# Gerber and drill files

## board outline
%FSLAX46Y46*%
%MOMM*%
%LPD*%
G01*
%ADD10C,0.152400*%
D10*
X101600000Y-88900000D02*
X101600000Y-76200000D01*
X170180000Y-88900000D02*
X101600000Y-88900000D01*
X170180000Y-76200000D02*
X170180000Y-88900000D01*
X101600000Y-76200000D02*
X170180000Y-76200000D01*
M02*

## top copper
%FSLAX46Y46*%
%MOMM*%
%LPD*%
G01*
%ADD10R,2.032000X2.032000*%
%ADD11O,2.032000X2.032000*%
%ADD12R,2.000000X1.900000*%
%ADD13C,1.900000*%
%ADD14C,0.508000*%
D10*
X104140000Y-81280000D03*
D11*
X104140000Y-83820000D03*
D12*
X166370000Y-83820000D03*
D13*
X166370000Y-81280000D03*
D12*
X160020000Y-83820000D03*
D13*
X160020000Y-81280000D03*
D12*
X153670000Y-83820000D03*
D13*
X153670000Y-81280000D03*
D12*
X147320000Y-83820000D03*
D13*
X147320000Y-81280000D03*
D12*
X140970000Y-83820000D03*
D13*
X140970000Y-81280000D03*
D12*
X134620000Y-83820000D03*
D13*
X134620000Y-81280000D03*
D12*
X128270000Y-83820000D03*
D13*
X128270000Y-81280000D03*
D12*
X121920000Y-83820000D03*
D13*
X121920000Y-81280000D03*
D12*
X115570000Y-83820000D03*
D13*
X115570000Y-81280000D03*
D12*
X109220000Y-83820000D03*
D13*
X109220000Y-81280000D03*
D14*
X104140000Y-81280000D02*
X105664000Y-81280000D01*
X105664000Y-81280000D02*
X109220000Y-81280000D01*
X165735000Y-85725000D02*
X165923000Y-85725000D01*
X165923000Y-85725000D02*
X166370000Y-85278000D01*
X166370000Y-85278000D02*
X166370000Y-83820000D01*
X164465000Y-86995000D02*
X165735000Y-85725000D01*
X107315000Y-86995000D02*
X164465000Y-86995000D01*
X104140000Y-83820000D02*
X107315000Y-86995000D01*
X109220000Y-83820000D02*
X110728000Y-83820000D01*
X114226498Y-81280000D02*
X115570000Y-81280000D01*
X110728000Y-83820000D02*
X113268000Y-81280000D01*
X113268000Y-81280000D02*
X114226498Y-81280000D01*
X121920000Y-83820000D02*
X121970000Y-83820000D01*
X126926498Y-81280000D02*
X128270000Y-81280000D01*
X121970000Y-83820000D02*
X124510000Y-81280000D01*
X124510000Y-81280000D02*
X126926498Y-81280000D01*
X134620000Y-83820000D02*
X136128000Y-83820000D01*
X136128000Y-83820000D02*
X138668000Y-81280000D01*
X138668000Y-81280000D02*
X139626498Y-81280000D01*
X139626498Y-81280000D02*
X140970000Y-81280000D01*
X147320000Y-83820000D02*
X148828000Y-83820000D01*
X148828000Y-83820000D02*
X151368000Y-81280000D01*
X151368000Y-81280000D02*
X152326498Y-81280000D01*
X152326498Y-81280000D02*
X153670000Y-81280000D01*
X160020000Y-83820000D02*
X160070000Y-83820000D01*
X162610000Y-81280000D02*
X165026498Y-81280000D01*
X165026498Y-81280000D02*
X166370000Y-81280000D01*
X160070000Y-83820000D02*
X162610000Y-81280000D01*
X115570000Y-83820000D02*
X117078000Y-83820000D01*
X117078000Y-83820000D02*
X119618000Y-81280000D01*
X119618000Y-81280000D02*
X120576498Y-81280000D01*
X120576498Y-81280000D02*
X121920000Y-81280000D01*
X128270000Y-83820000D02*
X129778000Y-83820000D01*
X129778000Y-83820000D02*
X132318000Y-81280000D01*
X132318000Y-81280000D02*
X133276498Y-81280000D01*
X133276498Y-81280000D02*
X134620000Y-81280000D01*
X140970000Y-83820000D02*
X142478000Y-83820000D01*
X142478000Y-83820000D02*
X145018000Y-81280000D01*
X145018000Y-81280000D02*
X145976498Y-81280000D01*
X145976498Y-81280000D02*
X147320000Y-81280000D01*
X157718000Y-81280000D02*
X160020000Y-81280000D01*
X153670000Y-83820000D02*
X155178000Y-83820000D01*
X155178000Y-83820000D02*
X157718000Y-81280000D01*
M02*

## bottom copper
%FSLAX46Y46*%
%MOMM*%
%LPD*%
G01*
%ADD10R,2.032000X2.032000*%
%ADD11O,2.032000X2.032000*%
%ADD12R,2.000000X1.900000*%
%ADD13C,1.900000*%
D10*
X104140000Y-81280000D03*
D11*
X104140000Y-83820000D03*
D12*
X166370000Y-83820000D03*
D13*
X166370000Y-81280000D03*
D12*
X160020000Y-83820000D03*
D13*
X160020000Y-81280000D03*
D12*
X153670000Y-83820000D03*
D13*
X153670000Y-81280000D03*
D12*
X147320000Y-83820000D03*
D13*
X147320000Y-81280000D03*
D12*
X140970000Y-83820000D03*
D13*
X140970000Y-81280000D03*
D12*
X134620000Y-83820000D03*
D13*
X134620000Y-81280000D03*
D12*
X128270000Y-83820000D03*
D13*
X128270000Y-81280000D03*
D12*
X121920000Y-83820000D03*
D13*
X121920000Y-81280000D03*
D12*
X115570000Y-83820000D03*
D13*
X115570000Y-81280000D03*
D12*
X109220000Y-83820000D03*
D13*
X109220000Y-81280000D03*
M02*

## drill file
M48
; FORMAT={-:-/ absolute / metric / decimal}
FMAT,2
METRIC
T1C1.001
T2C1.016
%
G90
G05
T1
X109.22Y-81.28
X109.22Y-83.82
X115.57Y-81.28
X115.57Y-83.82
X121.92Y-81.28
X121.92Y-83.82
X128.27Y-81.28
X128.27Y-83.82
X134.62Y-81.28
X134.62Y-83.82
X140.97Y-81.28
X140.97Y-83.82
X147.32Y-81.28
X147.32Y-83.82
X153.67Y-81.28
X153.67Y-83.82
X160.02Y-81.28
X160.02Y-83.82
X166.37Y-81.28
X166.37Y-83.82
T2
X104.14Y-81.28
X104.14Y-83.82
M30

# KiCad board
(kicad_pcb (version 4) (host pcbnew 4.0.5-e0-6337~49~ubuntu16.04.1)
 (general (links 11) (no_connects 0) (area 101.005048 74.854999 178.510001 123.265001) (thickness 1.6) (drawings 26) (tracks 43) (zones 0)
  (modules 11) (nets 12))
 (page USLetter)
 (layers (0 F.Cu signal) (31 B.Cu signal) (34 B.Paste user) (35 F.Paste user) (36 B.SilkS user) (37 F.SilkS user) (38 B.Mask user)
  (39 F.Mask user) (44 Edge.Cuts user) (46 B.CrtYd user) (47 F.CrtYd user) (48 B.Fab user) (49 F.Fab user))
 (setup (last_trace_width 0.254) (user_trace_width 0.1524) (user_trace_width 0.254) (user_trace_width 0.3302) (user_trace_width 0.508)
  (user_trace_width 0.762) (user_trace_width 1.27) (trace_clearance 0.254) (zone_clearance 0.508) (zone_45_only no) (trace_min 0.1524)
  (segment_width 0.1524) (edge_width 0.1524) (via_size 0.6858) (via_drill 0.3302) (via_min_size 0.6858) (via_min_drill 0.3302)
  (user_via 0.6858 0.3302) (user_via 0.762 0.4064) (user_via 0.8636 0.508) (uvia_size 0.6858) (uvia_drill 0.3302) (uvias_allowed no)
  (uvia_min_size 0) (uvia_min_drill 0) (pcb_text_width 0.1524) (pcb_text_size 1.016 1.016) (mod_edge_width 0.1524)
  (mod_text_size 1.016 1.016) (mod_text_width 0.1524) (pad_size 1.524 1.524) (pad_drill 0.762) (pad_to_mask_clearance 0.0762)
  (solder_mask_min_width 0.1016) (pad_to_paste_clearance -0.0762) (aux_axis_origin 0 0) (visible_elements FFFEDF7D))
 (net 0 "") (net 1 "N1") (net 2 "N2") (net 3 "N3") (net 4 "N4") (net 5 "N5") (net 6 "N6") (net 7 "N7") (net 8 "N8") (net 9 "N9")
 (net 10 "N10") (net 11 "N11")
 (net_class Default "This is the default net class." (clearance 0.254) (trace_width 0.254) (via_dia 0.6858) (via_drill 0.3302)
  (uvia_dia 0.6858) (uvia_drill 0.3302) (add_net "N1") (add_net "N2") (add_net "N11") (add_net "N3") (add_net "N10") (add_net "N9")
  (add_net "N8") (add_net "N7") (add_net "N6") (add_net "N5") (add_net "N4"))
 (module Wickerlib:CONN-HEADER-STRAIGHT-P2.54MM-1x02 (layer F.Cu) (at 104.14 81.28)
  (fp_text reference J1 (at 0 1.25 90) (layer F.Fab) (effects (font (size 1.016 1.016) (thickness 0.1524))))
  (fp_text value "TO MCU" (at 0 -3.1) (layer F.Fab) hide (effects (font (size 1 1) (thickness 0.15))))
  (pad 1 thru_hole rect (at 0 0) (size 2.032 2.032) (drill 1.016) (layers *.Cu *.Mask F.SilkS) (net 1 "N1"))
  (pad 2 thru_hole oval (at 0 2.54) (size 2.032 2.032) (drill 1.016) (layers *.Cu *.Mask F.SilkS) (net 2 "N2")))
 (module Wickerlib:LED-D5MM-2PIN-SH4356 (layer F.Cu) (at 166.37 83.82 90)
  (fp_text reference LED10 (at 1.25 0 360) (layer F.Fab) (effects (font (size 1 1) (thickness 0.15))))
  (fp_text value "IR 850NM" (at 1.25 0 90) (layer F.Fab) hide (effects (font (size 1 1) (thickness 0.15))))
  (pad 1 thru_hole rect (at 0 0 180) (size 2 1.9) (drill 1.00076) (layers *.Cu *.Mask F.SilkS) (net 2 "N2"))
  (pad 2 thru_hole circle (at 2.54 0 90) (size 1.9 1.9) (drill 1.00076) (layers *.Cu *.Mask F.SilkS) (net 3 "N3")))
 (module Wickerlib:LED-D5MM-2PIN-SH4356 (layer F.Cu) (at 160.02 83.82 90)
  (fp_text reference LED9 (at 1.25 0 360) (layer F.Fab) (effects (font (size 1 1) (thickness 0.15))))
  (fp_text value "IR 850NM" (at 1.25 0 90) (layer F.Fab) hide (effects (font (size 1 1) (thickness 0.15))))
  (pad 1 thru_hole rect (at 0 0 180) (size 2 1.9) (drill 1.00076) (layers *.Cu *.Mask F.SilkS) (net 3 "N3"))
  (pad 2 thru_hole circle (at 2.54 0 90) (size 1.9 1.9) (drill 1.00076) (layers *.Cu *.Mask F.SilkS) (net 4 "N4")))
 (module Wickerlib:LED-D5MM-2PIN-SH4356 (layer F.Cu) (at 153.67 83.82 90)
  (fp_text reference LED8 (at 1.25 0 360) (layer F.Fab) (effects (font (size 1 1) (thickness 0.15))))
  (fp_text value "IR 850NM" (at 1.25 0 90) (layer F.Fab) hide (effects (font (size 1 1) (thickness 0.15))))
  (pad 1 thru_hole rect (at 0 0 180) (size 2 1.9) (drill 1.00076) (layers *.Cu *.Mask F.SilkS) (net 4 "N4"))
  (pad 2 thru_hole circle (at 2.54 0 90) (size 1.9 1.9) (drill 1.00076) (layers *.Cu *.Mask F.SilkS) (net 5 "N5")))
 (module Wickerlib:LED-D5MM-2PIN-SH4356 (layer F.Cu) (at 147.32 83.82 90)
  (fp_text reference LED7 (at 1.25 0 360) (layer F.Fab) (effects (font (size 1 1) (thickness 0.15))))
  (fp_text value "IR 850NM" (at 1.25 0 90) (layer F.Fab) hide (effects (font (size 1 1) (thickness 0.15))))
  (pad 1 thru_hole rect (at 0 0 180) (size 2 1.9) (drill 1.00076) (layers *.Cu *.Mask F.SilkS) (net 5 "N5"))
  (pad 2 thru_hole circle (at 2.54 0 90) (size 1.9 1.9) (drill 1.00076) (layers *.Cu *.Mask F.SilkS) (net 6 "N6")))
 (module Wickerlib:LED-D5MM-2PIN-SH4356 (layer F.Cu) (at 140.97 83.82 90)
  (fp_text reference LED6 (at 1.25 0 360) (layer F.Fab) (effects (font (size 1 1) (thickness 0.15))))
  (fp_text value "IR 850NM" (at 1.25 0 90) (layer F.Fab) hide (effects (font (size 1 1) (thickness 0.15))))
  (pad 1 thru_hole rect (at 0 0 180) (size 2 1.9) (drill 1.00076) (layers *.Cu *.Mask F.SilkS) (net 6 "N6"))
  (pad 2 thru_hole circle (at 2.54 0 90) (size 1.9 1.9) (drill 1.00076) (layers *.Cu *.Mask F.SilkS) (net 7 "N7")))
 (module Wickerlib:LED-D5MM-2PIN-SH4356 (layer F.Cu) (at 134.62 83.82 90)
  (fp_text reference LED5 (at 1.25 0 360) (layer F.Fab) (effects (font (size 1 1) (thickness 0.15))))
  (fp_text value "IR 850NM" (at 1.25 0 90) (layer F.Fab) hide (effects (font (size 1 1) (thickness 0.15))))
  (pad 1 thru_hole rect (at 0 0 180) (size 2 1.9) (drill 1.00076) (layers *.Cu *.Mask F.SilkS) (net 7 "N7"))
  (pad 2 thru_hole circle (at 2.54 0 90) (size 1.9 1.9) (drill 1.00076) (layers *.Cu *.Mask F.SilkS) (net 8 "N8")))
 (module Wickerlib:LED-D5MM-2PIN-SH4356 (layer F.Cu) (at 128.27 83.82 90)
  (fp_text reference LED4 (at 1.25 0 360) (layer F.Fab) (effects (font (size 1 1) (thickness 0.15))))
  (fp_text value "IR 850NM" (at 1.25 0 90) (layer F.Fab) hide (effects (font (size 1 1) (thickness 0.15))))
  (pad 1 thru_hole rect (at 0 0 180) (size 2 1.9) (drill 1.00076) (layers *.Cu *.Mask F.SilkS) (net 8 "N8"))
  (pad 2 thru_hole circle (at 2.54 0 90) (size 1.9 1.9) (drill 1.00076) (layers *.Cu *.Mask F.SilkS) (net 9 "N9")))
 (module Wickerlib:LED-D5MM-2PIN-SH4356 (layer F.Cu) (at 121.92 83.82 90)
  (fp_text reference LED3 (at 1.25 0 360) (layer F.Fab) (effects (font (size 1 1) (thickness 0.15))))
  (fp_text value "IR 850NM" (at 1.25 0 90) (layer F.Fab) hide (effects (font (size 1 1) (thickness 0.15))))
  (pad 1 thru_hole rect (at 0 0 180) (size 2 1.9) (drill 1.00076) (layers *.Cu *.Mask F.SilkS) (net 9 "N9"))
  (pad 2 thru_hole circle (at 2.54 0 90) (size 1.9 1.9) (drill 1.00076) (layers *.Cu *.Mask F.SilkS) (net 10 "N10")))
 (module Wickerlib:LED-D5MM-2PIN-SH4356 (layer F.Cu) (at 115.57 83.82 90)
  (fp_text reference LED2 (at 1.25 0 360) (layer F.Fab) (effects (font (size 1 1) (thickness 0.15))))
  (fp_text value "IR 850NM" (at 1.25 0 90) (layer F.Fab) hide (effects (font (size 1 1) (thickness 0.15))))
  (pad 1 thru_hole rect (at 0 0 180) (size 2 1.9) (drill 1.00076) (layers *.Cu *.Mask F.SilkS) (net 10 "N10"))
  (pad 2 thru_hole circle (at 2.54 0 90) (size 1.9 1.9) (drill 1.00076) (layers *.Cu *.Mask F.SilkS) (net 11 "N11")))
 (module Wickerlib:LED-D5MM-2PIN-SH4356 (layer F.Cu) (at 109.22 83.82 90)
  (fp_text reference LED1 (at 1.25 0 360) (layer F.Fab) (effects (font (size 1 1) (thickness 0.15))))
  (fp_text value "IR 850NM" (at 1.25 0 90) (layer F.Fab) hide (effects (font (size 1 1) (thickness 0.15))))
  (pad 1 thru_hole rect (at 0 0 180) (size 2 1.9) (drill 1.00076) (layers *.Cu *.Mask F.SilkS) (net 11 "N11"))
  (pad 2 thru_hole circle (at 2.54 0 90) (size 1.9 1.9) (drill 1.00076) (layers *.Cu *.Mask F.SilkS) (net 1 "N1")))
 (gr_line (start 101.6 88.9) (end 101.6 76.2) (layer Edge.Cuts) (width 0.1524))
 (gr_line (start 170.18 88.9) (end 101.6 88.9) (layer Edge.Cuts) (width 0.1524))
 (gr_line (start 170.18 76.2) (end 170.18 88.9) (layer Edge.Cuts) (width 0.1524))
 (gr_line (start 101.6 76.2) (end 170.18 76.2) (layer Edge.Cuts) (width 0.1524))
 (segment (start 104.14 81.28) (end 105.664 81.28) (width 0.508) (layer F.Cu) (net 1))
 (segment (start 105.664 81.28) (end 109.22 81.28) (width 0.508) (layer F.Cu) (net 1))
 (segment (start 165.735 85.725) (end 165.923 85.725) (width 0.508) (layer F.Cu) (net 2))
 (segment (start 165.923 85.725) (end 166.37 85.278) (width 0.508) (layer F.Cu) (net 2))
 (segment (start 166.37 85.278) (end 166.37 83.82) (width 0.508) (layer F.Cu) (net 2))
 (segment (start 164.465 86.995) (end 165.735 85.725) (width 0.508) (layer F.Cu) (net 2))
 (segment (start 107.315 86.995) (end 164.465 86.995) (width 0.508) (layer F.Cu) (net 2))
 (segment (start 104.14 83.82) (end 107.315 86.995) (width 0.508) (layer F.Cu) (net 2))
 (segment (start 109.22 83.82) (end 110.728 83.82) (width 0.508) (layer F.Cu) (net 11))
 (segment (start 114.226498 81.28) (end 115.57 81.28) (width 0.508) (layer F.Cu) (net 11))
 (segment (start 110.728 83.82) (end 113.268 81.28) (width 0.508) (layer F.Cu) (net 11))
 (segment (start 113.268 81.28) (end 114.226498 81.28) (width 0.508) (layer F.Cu) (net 11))
 (segment (start 121.92 83.82) (end 121.97 83.82) (width 0.508) (layer F.Cu) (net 9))
 (segment (start 126.926498 81.28) (end 128.27 81.28) (width 0.508) (layer F.Cu) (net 9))
 (segment (start 121.97 83.82) (end 124.51 81.28) (width 0.508) (layer F.Cu) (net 9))
 (segment (start 124.51 81.28) (end 126.926498 81.28) (width 0.508) (layer F.Cu) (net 9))
 (segment (start 134.62 83.82) (end 136.128 83.82) (width 0.508) (layer F.Cu) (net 7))
 (segment (start 136.128 83.82) (end 138.668 81.28) (width 0.508) (layer F.Cu) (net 7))
 (segment (start 138.668 81.28) (end 139.626498 81.28) (width 0.508) (layer F.Cu) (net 7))
 (segment (start 139.626498 81.28) (end 140.97 81.28) (width 0.508) (layer F.Cu) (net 7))
 (segment (start 147.32 83.82) (end 148.828 83.82) (width 0.508) (layer F.Cu) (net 5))
 (segment (start 148.828 83.82) (end 151.368 81.28) (width 0.508) (layer F.Cu) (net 5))
 (segment (start 151.368 81.28) (end 152.326498 81.28) (width 0.508) (layer F.Cu) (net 5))
 (segment (start 152.326498 81.28) (end 153.67 81.28) (width 0.508) (layer F.Cu) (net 5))
 (segment (start 160.02 83.82) (end 160.07 83.82) (width 0.508) (layer F.Cu) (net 3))
 (segment (start 162.61 81.28) (end 165.026498 81.28) (width 0.508) (layer F.Cu) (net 3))
 (segment (start 165.026498 81.28) (end 166.37 81.28) (width 0.508) (layer F.Cu) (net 3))
 (segment (start 160.07 83.82) (end 162.61 81.28) (width 0.508) (layer F.Cu) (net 3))
 (segment (start 115.57 83.82) (end 117.078 83.82) (width 0.508) (layer F.Cu) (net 10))
 (segment (start 117.078 83.82) (end 119.618 81.28) (width 0.508) (layer F.Cu) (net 10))
 (segment (start 119.618 81.28) (end 120.576498 81.28) (width 0.508) (layer F.Cu) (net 10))
 (segment (start 120.576498 81.28) (end 121.92 81.28) (width 0.508) (layer F.Cu) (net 10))
 (segment (start 128.27 83.82) (end 129.778 83.82) (width 0.508) (layer F.Cu) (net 8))
 (segment (start 129.778 83.82) (end 132.318 81.28) (width 0.508) (layer F.Cu) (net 8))
 (segment (start 132.318 81.28) (end 133.276498 81.28) (width 0.508) (layer F.Cu) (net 8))
 (segment (start 133.276498 81.28) (end 134.62 81.28) (width 0.508) (layer F.Cu) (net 8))
 (segment (start 140.97 83.82) (end 142.478 83.82) (width 0.508) (layer F.Cu) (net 6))
 (segment (start 142.478 83.82) (end 145.018 81.28) (width 0.508) (layer F.Cu) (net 6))
 (segment (start 145.018 81.28) (end 145.976498 81.28) (width 0.508) (layer F.Cu) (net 6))
 (segment (start 145.976498 81.28) (end 147.32 81.28) (width 0.508) (layer F.Cu) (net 6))
 (segment (start 157.718 81.28) (end 160.02 81.28) (width 0.508) (layer F.Cu) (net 4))
 (segment (start 153.67 83.82) (end 155.178 83.82) (width 0.508) (layer F.Cu) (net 4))
 (segment (start 155.178 83.82) (end 157.718 81.28) (width 0.508) (layer F.Cu) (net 4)))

